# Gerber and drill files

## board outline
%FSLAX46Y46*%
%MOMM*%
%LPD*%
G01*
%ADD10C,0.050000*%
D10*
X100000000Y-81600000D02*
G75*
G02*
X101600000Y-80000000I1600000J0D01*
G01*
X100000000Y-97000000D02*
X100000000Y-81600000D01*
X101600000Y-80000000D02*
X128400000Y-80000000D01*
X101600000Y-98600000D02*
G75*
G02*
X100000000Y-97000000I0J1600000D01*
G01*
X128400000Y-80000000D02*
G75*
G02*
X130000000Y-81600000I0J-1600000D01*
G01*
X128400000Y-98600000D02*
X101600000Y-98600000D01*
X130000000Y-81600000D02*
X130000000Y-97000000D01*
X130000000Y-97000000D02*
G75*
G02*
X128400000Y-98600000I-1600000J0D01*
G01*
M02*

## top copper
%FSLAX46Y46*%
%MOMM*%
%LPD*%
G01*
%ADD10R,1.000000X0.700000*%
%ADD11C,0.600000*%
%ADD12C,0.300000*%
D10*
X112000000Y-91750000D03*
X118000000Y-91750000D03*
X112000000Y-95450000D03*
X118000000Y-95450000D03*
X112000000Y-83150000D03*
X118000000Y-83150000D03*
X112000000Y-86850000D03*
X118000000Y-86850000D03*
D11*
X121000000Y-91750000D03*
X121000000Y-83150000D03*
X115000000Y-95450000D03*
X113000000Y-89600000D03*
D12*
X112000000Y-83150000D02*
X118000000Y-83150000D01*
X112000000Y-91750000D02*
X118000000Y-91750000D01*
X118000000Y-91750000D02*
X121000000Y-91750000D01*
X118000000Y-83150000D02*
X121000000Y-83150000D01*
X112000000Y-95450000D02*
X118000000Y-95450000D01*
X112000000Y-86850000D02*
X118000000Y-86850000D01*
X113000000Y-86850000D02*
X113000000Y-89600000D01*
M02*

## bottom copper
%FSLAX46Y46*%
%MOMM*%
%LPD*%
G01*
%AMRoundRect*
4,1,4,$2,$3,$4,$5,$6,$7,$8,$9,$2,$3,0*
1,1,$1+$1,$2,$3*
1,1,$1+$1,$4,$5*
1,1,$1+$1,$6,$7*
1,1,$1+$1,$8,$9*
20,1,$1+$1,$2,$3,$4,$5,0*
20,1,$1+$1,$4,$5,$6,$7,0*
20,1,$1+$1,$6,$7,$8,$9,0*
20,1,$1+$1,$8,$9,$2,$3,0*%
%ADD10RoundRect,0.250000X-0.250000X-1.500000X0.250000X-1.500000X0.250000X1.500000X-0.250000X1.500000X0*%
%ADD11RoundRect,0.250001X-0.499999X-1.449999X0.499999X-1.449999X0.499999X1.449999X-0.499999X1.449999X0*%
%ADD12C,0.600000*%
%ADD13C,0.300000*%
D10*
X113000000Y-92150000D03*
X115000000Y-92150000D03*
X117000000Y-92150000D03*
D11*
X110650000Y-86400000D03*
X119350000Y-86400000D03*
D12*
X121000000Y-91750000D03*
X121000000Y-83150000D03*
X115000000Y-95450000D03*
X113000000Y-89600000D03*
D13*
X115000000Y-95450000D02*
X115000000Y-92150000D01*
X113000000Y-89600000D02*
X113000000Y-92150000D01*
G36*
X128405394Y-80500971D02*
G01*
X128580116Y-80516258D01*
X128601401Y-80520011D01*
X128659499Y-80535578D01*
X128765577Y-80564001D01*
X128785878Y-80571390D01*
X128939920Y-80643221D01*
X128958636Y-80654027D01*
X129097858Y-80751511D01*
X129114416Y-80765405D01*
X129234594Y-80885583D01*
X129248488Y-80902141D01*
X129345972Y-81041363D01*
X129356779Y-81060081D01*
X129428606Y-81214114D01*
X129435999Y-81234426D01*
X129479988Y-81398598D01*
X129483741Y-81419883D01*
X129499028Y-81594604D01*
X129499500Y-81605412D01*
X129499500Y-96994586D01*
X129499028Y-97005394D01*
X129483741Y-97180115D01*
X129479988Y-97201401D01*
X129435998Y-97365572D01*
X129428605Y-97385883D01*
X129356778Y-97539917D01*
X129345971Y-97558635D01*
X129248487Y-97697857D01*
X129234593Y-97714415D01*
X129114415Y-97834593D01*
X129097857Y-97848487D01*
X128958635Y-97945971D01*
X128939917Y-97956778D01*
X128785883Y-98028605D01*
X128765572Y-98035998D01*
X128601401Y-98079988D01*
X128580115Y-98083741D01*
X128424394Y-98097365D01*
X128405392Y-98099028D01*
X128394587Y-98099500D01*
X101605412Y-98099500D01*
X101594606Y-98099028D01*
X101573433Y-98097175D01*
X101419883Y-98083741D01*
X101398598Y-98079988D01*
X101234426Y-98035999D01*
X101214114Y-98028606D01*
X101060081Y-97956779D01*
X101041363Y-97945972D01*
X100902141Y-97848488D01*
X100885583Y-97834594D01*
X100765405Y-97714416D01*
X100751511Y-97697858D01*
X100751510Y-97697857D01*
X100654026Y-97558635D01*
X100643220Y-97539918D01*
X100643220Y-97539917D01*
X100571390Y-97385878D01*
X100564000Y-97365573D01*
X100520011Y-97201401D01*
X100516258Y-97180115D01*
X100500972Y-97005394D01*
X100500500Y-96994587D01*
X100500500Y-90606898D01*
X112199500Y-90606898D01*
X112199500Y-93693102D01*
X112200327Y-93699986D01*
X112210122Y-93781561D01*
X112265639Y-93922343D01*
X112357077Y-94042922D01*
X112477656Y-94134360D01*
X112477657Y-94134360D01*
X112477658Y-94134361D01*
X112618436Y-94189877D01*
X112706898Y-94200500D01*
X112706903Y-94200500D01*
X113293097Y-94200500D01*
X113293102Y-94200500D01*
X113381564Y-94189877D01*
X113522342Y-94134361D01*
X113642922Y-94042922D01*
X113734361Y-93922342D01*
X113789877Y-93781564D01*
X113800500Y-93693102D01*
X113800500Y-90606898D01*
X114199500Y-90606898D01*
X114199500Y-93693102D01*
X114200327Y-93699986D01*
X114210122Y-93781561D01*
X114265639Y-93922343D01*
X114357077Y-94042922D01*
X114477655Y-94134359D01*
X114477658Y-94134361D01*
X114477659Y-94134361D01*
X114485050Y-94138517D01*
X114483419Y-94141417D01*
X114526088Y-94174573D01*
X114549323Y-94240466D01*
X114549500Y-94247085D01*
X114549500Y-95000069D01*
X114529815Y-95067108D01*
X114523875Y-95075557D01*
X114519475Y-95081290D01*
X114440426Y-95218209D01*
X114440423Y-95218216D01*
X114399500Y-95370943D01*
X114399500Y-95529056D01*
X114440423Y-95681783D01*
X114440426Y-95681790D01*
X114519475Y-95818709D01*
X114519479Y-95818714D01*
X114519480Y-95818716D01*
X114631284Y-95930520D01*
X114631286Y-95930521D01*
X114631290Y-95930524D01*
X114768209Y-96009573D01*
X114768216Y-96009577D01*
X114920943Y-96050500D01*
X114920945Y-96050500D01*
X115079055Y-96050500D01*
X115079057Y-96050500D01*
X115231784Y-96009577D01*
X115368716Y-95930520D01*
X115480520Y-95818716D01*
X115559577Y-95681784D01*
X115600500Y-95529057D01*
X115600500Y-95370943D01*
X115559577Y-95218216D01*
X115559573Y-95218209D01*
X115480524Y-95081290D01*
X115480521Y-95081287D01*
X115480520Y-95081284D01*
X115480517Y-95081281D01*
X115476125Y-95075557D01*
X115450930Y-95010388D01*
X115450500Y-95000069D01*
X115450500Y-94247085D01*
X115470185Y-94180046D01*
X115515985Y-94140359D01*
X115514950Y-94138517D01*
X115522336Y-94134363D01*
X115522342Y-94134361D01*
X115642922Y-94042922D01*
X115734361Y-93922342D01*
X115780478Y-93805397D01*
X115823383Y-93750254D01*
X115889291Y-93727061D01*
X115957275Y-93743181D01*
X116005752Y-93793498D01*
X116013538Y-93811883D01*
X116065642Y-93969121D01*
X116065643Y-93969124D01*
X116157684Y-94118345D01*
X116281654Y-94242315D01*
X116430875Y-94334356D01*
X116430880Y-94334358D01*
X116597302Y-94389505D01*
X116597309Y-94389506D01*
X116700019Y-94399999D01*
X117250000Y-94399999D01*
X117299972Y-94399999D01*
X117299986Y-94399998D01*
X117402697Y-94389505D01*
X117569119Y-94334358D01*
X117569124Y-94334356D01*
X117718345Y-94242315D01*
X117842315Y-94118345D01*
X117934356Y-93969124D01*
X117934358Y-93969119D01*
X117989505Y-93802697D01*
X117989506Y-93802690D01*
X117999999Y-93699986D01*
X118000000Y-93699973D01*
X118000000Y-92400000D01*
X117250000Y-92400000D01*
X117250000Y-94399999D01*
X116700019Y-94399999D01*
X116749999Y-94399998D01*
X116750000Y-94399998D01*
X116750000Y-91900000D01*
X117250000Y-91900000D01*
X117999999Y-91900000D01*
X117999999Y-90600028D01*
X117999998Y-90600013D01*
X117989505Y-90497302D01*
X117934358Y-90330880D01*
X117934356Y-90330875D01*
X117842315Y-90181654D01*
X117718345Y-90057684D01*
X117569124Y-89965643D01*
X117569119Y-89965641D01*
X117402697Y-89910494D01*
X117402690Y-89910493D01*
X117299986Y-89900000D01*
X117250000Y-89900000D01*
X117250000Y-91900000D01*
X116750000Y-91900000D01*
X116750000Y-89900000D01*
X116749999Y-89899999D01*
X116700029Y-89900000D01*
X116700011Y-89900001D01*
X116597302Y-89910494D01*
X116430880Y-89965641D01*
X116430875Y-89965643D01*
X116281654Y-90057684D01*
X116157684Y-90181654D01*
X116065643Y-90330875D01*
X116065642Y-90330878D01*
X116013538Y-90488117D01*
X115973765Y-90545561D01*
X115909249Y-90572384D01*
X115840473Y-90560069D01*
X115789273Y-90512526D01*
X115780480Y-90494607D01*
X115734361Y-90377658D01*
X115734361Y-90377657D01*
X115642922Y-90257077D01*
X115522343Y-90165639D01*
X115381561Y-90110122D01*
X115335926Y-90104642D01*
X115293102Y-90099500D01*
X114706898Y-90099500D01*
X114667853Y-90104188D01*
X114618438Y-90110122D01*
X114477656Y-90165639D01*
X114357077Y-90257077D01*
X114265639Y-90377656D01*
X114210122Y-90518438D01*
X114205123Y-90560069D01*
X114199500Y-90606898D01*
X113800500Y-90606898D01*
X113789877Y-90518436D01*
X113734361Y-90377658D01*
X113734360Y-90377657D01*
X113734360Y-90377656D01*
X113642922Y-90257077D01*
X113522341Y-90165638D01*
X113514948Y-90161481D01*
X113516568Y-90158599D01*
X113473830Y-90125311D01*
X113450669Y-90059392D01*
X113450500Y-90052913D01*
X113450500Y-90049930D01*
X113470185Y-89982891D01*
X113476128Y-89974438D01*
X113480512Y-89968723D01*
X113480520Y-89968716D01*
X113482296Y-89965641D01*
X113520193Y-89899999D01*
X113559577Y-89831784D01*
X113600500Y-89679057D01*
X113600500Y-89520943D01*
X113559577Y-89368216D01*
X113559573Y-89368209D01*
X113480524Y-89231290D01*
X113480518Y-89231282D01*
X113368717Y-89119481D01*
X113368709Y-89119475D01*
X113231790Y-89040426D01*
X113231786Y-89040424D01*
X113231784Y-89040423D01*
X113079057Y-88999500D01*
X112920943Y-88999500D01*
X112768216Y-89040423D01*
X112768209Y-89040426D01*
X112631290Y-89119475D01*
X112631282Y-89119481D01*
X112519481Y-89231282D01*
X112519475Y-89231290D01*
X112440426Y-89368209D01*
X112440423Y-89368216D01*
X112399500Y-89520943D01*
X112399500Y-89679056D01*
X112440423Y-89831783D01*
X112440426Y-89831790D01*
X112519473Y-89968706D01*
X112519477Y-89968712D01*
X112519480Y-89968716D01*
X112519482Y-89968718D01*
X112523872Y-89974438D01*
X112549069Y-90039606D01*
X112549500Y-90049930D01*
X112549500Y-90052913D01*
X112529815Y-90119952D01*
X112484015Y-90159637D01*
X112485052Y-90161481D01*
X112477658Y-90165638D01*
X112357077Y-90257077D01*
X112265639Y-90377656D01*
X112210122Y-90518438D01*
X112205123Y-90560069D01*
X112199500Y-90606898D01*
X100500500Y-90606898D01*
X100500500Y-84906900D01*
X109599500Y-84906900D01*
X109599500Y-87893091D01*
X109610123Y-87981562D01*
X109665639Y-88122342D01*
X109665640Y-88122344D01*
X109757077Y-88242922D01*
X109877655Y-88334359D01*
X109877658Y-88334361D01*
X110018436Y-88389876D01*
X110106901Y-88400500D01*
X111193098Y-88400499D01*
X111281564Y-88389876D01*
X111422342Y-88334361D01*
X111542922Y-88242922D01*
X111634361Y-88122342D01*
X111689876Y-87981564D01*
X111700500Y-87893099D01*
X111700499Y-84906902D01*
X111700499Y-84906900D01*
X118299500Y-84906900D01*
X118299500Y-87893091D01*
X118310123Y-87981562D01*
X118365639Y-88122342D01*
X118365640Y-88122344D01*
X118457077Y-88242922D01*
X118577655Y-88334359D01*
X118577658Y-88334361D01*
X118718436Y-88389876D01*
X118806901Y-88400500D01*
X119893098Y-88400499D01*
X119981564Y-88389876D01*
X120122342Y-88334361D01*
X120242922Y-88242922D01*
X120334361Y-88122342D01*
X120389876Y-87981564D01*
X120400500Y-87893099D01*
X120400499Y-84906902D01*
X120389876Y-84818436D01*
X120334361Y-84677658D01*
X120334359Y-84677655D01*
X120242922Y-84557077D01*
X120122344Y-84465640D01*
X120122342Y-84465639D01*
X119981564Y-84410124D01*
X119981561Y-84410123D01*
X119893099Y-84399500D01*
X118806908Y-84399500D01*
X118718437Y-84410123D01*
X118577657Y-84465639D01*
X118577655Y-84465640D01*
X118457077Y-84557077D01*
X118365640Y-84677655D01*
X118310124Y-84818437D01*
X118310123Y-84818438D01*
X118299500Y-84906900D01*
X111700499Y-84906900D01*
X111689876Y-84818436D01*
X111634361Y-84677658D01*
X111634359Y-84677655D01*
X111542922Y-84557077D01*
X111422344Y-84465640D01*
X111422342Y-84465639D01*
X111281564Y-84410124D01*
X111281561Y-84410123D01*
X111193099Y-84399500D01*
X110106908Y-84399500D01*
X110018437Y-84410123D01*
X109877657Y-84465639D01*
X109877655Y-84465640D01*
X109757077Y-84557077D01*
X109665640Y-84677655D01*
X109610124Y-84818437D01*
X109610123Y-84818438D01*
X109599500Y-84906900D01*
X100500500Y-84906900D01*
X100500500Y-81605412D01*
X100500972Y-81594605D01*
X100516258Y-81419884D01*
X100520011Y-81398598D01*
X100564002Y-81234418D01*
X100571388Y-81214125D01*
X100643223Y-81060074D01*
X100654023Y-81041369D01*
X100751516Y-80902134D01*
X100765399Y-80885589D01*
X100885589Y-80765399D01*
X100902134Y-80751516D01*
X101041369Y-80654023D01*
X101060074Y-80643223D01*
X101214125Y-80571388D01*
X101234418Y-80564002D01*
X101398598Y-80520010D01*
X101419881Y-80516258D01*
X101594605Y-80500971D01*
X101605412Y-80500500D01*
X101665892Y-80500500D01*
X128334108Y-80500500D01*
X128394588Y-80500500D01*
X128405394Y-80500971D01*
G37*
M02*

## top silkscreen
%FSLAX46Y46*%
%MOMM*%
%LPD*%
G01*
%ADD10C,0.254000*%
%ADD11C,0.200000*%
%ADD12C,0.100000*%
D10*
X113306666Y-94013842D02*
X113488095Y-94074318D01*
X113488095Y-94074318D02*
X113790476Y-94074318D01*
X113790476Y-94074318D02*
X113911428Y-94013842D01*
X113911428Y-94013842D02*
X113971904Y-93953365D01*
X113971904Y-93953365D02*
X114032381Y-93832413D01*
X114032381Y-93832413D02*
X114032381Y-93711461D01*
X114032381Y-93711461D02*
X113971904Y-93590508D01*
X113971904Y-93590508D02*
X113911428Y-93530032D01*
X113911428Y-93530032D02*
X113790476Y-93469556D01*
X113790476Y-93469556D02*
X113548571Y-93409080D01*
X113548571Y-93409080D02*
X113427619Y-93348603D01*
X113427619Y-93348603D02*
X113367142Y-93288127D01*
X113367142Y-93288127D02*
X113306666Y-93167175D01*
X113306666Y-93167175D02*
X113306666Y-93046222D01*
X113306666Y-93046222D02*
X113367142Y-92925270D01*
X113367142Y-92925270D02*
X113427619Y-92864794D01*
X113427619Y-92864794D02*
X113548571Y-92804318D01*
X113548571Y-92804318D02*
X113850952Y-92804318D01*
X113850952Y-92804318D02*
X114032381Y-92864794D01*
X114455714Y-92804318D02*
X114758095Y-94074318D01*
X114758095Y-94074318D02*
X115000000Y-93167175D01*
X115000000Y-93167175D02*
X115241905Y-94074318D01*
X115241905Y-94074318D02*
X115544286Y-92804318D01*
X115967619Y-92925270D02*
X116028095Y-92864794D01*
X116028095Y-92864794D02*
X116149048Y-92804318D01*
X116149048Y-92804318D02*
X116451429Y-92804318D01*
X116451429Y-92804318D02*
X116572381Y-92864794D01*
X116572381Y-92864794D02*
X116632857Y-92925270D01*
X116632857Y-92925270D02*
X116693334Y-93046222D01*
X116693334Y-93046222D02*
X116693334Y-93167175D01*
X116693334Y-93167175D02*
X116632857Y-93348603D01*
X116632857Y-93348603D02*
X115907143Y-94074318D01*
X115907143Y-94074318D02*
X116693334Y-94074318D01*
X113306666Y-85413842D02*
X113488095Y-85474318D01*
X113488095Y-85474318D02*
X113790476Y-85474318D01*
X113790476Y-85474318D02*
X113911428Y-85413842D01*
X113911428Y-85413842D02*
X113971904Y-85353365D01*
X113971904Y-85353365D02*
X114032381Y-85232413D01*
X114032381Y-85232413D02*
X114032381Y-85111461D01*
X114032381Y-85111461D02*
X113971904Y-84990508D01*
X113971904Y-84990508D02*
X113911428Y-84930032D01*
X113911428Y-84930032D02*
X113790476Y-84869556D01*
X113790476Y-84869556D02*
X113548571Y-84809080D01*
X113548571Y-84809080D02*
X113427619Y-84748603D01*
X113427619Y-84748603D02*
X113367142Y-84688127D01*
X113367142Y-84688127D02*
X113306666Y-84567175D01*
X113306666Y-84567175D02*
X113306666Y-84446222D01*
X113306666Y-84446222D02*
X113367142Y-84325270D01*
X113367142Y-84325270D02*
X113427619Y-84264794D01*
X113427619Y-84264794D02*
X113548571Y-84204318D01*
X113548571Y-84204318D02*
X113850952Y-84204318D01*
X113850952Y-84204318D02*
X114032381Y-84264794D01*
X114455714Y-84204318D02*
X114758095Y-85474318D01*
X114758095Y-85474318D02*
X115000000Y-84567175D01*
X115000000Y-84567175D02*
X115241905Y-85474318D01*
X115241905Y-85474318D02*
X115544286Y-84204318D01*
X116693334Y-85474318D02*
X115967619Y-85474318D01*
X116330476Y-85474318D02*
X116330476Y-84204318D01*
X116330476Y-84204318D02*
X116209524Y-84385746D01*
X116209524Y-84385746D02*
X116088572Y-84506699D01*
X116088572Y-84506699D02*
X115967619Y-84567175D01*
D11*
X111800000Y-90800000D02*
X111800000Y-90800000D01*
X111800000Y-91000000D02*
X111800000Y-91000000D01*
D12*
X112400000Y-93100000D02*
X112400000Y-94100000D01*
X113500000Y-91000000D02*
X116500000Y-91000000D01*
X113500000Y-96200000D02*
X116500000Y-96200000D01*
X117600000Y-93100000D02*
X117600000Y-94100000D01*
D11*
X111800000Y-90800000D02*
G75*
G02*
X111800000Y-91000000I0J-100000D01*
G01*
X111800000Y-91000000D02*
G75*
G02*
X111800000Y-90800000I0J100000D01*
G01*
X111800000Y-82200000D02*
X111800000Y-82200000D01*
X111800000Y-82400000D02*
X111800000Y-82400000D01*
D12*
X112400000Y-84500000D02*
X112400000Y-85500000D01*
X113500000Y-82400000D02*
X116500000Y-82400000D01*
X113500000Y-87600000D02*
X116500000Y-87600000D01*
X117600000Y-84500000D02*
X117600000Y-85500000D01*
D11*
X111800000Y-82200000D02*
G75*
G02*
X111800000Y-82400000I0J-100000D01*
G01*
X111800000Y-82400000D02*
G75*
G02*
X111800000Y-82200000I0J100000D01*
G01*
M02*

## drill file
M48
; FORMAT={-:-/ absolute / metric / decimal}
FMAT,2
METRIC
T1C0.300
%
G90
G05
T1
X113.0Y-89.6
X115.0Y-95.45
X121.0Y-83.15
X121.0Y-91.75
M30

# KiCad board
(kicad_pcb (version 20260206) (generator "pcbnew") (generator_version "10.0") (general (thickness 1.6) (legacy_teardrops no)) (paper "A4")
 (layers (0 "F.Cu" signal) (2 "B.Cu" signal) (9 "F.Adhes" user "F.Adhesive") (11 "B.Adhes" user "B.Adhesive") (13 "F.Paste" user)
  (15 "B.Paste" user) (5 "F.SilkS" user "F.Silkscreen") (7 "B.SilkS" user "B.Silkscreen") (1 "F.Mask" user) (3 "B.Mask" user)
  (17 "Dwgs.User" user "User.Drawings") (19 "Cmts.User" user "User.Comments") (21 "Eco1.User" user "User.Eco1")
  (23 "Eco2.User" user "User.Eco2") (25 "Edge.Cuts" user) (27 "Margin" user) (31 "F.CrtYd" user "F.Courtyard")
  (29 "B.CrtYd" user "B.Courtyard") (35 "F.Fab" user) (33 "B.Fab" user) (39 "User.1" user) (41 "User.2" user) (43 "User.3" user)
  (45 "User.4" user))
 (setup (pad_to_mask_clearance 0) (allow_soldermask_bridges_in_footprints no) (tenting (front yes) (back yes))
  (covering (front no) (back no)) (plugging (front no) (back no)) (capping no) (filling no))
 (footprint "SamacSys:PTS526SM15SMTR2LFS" (layer "F.Cu") (at 115 93.6)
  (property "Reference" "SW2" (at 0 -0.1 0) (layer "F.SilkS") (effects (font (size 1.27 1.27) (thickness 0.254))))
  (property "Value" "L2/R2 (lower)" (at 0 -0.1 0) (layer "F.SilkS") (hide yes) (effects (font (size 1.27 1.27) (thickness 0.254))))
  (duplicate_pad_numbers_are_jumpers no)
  (fp_line (start -3.2 -2.8) (end -3.2 -2.8) (stroke (width 0.2) (type solid)) (layer "F.SilkS"))
  (fp_line (start -3.2 -2.6) (end -3.2 -2.6) (stroke (width 0.2) (type solid)) (layer "F.SilkS"))
  (fp_line (start -2.6 -0.5) (end -2.6 0.5) (stroke (width 0.1) (type solid)) (layer "F.SilkS"))
  (fp_line (start -1.5 -2.6) (end 1.5 -2.6) (stroke (width 0.1) (type solid)) (layer "F.SilkS"))
  (fp_line (start -1.5 2.6) (end 1.5 2.6) (stroke (width 0.1) (type solid)) (layer "F.SilkS"))
  (fp_line (start 2.6 -0.5) (end 2.6 0.5) (stroke (width 0.1) (type solid)) (layer "F.SilkS"))
  (fp_arc (start -3.2 -2.8) (mid -3.1 -2.7) (end -3.2 -2.6) (stroke (width 0.2) (type solid)) (layer "F.SilkS"))
  (fp_arc (start -3.2 -2.6) (mid -3.3 -2.7) (end -3.2 -2.8) (stroke (width 0.2) (type solid)) (layer "F.SilkS"))
  (pad "1" smd rect (at -3 -1.85 90) (size 0.7 1) (layers "F.Cu" "F.Mask" "F.Paste") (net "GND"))
  (pad "2" smd rect (at 3 -1.85 90) (size 0.7 1) (layers "F.Cu" "F.Mask" "F.Paste") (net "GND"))
  (pad "3" smd rect (at -3 1.85 90) (size 0.7 1) (layers "F.Cu" "F.Mask" "F.Paste") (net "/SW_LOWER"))
  (pad "4" smd rect (at 3 1.85 90) (size 0.7 1) (layers "F.Cu" "F.Mask" "F.Paste") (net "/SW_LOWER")))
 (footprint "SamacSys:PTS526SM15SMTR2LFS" (layer "F.Cu") (at 115 85)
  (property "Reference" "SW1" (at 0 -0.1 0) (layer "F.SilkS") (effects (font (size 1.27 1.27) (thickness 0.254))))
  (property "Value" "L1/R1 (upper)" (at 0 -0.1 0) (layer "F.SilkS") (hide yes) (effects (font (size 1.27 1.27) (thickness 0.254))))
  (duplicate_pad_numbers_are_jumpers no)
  (fp_line (start -3.2 -2.8) (end -3.2 -2.8) (stroke (width 0.2) (type solid)) (layer "F.SilkS"))
  (fp_line (start -3.2 -2.6) (end -3.2 -2.6) (stroke (width 0.2) (type solid)) (layer "F.SilkS"))
  (fp_line (start -2.6 -0.5) (end -2.6 0.5) (stroke (width 0.1) (type solid)) (layer "F.SilkS"))
  (fp_line (start -1.5 -2.6) (end 1.5 -2.6) (stroke (width 0.1) (type solid)) (layer "F.SilkS"))
  (fp_line (start -1.5 2.6) (end 1.5 2.6) (stroke (width 0.1) (type solid)) (layer "F.SilkS"))
  (fp_line (start 2.6 -0.5) (end 2.6 0.5) (stroke (width 0.1) (type solid)) (layer "F.SilkS"))
  (fp_arc (start -3.2 -2.8) (mid -3.1 -2.7) (end -3.2 -2.6) (stroke (width 0.2) (type solid)) (layer "F.SilkS"))
  (fp_arc (start -3.2 -2.6) (mid -3.3 -2.7) (end -3.2 -2.8) (stroke (width 0.2) (type solid)) (layer "F.SilkS"))
  (pad "1" smd rect (at -3 -1.85 90) (size 0.7 1) (layers "F.Cu" "F.Mask" "F.Paste") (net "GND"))
  (pad "2" smd rect (at 3 -1.85 90) (size 0.7 1) (layers "F.Cu" "F.Mask" "F.Paste") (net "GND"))
  (pad "3" smd rect (at -3 1.85 90) (size 0.7 1) (layers "F.Cu" "F.Mask" "F.Paste") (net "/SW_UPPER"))
  (pad "4" smd rect (at 3 1.85 90) (size 0.7 1) (layers "F.Cu" "F.Mask" "F.Paste") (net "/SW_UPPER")))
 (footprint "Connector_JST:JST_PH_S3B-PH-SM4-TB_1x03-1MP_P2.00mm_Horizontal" (layer "B.Cu") (at 115 89.3)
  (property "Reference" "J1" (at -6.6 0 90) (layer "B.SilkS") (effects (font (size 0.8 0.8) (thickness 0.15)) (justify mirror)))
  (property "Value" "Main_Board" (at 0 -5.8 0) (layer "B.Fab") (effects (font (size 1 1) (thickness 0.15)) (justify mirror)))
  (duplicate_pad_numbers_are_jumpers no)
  (pad "1" smd roundrect (at -2 2.85) (size 1 3.5) (layers "B.Cu" "B.Mask" "B.Paste") (roundrect_rratio 0.25) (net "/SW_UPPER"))
  (pad "2" smd roundrect (at 0 2.85) (size 1 3.5) (layers "B.Cu" "B.Mask" "B.Paste") (roundrect_rratio 0.25) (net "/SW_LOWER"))
  (pad "3" smd roundrect (at 2 2.85) (size 1 3.5) (layers "B.Cu" "B.Mask" "B.Paste") (roundrect_rratio 0.25) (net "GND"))
  (pad "MP" smd roundrect (at -4.35 -2.9) (size 1.5 3.4) (layers "B.Cu" "B.Mask" "B.Paste") (roundrect_rratio 0.166667))
  (pad "MP" smd roundrect (at 4.35 -2.9) (size 1.5 3.4) (layers "B.Cu" "B.Mask" "B.Paste") (roundrect_rratio 0.166667)))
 (gr_arc (start 100 81.6) (mid 100.468629 80.468629) (end 101.6 80) (stroke (width 0.05) (type default)) (layer "Edge.Cuts"))
 (gr_line (start 100 97) (end 100 81.6) (stroke (width 0.05) (type default)) (layer "Edge.Cuts"))
 (gr_line (start 101.6 80) (end 128.4 80) (stroke (width 0.05) (type default)) (layer "Edge.Cuts"))
 (gr_arc (start 101.6 98.6) (mid 100.468629 98.13137) (end 100 97) (stroke (width 0.05) (type default)) (layer "Edge.Cuts"))
 (gr_arc (start 128.4 80) (mid 129.53137 80.468629) (end 130 81.6) (stroke (width 0.05) (type default)) (layer "Edge.Cuts"))
 (gr_line (start 128.4 98.6) (end 101.6 98.6) (stroke (width 0.05) (type default)) (layer "Edge.Cuts"))
 (gr_line (start 130 81.6) (end 130 97) (stroke (width 0.05) (type default)) (layer "Edge.Cuts"))
 (gr_arc (start 130 97) (mid 129.53137 98.13137) (end 128.4 98.6) (stroke (width 0.05) (type default)) (layer "Edge.Cuts"))
 (segment (start 112 83.15) (end 118 83.15) (width 0.3) (layer "F.Cu") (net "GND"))
 (segment (start 112 91.75) (end 118 91.75) (width 0.3) (layer "F.Cu") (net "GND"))
 (segment (start 118 91.75) (end 121 91.75) (width 0.3) (layer "F.Cu") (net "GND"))
 (segment (start 118 83.15) (end 121 83.15) (width 0.3) (layer "F.Cu") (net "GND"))
 (via (at 121 91.75) (size 0.6) (drill 0.3) (layers "F.Cu" "B.Cu") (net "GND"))
 (via (at 121 83.15) (size 0.6) (drill 0.3) (layers "F.Cu" "B.Cu") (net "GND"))
 (segment (start 112 95.45) (end 118 95.45) (width 0.3) (layer "F.Cu") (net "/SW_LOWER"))
 (via (at 115 95.45) (size 0.6) (drill 0.3) (layers "F.Cu" "B.Cu") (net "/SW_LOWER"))
 (segment (start 115 95.45) (end 115 92.15) (width 0.3) (layer "B.Cu") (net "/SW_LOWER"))
 (segment (start 112 86.85) (end 118 86.85) (width 0.3) (layer "F.Cu") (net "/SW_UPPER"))
 (segment (start 113 86.85) (end 113 89.6) (width 0.3) (layer "F.Cu") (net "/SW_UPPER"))
 (via (at 113 89.6) (size 0.6) (drill 0.3) (layers "F.Cu" "B.Cu") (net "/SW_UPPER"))
 (segment (start 113 89.6) (end 113 92.15) (width 0.3) (layer "B.Cu") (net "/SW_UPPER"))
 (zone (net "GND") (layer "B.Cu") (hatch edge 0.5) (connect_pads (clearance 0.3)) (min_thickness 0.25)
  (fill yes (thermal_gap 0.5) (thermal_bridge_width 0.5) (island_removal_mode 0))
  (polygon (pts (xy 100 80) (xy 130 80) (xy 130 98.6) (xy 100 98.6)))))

